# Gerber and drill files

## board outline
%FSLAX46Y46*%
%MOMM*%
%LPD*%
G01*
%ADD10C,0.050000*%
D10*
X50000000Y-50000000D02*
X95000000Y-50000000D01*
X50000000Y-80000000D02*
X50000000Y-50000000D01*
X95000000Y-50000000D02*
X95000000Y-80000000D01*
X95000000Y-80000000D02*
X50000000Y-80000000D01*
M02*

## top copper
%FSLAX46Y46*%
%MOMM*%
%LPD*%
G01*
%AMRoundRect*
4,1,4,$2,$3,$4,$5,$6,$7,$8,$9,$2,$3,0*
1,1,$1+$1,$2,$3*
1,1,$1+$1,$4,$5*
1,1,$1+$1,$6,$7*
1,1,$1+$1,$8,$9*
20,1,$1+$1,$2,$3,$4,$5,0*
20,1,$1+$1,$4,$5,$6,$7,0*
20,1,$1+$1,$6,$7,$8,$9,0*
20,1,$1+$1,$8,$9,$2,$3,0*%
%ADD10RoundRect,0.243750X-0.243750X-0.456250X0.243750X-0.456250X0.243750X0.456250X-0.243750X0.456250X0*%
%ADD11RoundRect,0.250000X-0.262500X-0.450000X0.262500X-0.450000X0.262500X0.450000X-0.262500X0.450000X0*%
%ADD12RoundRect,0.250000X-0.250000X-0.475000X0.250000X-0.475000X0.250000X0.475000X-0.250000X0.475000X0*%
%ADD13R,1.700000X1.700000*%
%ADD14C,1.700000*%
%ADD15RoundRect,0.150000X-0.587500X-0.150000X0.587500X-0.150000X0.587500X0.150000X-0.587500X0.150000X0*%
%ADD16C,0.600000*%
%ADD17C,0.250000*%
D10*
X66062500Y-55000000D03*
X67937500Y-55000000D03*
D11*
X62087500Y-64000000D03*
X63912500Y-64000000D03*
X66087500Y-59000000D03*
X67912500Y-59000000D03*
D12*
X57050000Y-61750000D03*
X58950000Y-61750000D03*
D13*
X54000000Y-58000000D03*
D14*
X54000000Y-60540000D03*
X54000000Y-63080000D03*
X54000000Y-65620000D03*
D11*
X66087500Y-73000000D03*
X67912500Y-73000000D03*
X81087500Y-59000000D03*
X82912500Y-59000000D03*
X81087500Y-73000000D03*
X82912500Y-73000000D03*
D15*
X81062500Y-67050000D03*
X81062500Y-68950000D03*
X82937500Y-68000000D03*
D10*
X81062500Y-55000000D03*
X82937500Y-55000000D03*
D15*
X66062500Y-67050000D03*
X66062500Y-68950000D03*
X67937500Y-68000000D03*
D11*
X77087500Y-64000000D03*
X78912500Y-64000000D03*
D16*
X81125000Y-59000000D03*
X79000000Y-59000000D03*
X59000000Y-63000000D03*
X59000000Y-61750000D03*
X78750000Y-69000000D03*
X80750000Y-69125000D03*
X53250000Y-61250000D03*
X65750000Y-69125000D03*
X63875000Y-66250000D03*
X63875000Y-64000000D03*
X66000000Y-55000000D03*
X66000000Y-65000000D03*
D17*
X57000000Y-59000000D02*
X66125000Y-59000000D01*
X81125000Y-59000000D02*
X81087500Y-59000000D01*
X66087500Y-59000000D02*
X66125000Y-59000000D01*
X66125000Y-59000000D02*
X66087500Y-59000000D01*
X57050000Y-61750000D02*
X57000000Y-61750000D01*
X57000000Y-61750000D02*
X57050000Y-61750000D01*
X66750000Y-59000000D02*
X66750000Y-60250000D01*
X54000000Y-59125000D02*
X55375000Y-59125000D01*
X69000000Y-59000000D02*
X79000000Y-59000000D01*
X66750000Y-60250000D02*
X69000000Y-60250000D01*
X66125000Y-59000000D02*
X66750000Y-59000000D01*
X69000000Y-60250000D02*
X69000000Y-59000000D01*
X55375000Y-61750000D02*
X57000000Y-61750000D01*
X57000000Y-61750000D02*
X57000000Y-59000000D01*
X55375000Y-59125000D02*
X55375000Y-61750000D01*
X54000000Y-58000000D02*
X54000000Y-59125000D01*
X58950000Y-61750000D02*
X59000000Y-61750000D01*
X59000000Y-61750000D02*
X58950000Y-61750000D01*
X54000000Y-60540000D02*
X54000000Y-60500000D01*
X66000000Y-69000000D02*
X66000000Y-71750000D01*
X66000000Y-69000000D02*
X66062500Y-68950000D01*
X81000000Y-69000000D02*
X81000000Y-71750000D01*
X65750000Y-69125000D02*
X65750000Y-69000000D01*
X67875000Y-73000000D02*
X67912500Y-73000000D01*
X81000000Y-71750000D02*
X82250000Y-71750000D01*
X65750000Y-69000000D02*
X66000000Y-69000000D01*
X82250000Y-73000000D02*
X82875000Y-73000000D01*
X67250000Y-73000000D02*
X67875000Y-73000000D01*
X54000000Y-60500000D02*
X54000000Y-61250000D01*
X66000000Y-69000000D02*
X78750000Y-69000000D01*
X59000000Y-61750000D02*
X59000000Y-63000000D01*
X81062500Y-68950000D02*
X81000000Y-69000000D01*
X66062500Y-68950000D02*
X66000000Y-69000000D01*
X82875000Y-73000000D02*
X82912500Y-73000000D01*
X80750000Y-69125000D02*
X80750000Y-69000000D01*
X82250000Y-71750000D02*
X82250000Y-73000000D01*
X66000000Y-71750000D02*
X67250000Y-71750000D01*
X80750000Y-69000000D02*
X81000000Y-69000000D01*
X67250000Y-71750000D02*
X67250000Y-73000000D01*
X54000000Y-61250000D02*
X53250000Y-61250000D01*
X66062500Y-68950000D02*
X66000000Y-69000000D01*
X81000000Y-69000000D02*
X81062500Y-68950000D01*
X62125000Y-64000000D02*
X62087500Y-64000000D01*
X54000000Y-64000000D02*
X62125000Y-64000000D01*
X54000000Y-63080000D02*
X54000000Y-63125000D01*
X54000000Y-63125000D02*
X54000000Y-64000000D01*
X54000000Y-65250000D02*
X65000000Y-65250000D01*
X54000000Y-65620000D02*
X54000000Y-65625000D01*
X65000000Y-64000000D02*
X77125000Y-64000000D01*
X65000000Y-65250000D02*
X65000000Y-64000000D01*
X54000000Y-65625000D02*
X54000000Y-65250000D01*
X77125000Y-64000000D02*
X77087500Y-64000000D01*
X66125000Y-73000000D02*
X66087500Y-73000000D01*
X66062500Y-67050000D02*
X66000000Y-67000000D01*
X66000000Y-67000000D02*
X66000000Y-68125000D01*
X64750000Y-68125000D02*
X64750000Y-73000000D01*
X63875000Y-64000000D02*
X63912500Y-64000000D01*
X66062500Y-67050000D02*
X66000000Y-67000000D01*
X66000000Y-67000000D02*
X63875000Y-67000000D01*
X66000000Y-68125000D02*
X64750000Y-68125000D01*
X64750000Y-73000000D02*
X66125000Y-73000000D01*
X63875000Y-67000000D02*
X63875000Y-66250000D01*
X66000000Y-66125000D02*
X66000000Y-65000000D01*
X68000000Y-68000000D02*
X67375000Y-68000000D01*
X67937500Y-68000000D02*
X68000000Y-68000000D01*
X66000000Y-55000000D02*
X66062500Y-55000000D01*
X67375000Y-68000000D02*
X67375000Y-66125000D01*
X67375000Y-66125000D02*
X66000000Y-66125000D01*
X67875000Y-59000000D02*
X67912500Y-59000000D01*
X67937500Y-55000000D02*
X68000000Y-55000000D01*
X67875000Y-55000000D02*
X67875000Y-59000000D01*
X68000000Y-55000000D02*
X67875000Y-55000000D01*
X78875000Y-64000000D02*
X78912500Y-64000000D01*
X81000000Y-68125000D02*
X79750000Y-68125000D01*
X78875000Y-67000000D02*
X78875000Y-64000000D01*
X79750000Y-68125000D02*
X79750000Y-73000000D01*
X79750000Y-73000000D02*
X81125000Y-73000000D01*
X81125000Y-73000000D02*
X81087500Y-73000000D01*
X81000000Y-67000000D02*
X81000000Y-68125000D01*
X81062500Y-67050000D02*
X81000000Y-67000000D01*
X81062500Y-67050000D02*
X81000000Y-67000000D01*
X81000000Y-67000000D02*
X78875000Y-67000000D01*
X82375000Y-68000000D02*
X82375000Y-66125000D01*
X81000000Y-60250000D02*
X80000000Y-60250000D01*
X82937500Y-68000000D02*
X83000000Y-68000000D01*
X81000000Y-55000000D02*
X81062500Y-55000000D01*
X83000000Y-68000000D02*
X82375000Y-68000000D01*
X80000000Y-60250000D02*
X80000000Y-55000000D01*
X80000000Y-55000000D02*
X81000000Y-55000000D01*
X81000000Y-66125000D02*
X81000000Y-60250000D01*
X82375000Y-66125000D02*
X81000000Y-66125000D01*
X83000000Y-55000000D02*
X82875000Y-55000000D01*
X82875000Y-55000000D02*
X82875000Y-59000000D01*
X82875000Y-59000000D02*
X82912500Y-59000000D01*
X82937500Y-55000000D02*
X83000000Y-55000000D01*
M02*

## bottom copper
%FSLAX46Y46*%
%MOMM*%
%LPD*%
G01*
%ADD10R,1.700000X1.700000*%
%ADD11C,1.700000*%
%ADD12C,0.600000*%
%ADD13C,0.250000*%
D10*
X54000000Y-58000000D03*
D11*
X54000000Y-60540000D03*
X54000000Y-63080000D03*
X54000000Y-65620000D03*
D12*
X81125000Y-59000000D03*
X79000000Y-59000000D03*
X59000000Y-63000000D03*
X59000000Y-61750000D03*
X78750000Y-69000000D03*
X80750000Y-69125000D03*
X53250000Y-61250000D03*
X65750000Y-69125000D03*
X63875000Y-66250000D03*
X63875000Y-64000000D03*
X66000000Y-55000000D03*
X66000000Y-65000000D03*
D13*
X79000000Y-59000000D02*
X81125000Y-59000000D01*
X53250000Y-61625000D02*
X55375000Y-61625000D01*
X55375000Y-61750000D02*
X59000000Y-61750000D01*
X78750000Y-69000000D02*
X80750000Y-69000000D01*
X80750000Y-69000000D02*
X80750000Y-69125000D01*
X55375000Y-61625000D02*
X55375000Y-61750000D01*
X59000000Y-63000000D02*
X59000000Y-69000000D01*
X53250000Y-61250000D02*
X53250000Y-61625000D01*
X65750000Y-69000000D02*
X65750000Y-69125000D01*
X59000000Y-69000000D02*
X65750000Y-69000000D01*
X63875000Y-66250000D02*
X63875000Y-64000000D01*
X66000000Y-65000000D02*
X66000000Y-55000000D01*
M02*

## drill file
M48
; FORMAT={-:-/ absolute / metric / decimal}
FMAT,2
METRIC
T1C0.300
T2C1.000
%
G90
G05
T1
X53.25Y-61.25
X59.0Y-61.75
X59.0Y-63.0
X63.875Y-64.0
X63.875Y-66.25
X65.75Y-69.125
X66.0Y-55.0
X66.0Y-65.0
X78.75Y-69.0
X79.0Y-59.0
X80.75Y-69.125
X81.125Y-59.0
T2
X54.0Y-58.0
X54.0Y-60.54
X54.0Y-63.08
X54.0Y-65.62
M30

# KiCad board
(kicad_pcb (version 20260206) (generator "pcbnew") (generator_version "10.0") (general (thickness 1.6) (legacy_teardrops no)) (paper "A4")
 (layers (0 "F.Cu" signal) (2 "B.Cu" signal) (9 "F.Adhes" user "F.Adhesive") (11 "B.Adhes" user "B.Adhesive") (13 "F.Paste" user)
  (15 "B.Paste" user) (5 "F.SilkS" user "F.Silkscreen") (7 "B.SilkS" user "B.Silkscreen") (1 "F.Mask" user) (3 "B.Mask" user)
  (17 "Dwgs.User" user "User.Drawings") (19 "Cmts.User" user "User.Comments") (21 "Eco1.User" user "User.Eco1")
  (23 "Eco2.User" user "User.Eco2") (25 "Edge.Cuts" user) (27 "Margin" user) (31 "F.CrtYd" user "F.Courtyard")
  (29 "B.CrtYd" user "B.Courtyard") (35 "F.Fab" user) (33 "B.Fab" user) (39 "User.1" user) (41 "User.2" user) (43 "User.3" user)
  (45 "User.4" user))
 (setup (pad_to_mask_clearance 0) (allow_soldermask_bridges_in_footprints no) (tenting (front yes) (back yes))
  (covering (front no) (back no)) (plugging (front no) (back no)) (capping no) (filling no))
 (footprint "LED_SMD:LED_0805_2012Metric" (layer "F.Cu") (at 67 55)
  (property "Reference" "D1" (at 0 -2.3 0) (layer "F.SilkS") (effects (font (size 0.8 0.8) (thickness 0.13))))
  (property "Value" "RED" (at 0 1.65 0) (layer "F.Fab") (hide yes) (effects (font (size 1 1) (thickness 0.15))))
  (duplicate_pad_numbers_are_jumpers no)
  (pad "1" smd roundrect (at -0.9375 0) (size 0.975 1.4) (layers "F.Cu" "F.Mask" "F.Paste") (roundrect_rratio 0.25) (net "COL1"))
  (pad "2" smd roundrect (at 0.9375 0) (size 0.975 1.4) (layers "F.Cu" "F.Mask" "F.Paste") (roundrect_rratio 0.25) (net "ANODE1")))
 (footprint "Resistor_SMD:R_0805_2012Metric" (layer "F.Cu") (at 63 64)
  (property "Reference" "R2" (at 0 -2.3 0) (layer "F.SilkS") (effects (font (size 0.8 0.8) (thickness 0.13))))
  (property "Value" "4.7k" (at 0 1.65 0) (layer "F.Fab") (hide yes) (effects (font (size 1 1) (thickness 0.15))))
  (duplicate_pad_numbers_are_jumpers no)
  (pad "1" smd roundrect (at -0.9125 0) (size 1.025 1.4) (layers "F.Cu" "F.Mask" "F.Paste") (roundrect_rratio 0.243902) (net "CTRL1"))
  (pad "2" smd roundrect (at 0.9125 0) (size 1.025 1.4) (layers "F.Cu" "F.Mask" "F.Paste") (roundrect_rratio 0.243902) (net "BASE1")))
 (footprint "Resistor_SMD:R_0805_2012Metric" (layer "F.Cu") (at 67 59)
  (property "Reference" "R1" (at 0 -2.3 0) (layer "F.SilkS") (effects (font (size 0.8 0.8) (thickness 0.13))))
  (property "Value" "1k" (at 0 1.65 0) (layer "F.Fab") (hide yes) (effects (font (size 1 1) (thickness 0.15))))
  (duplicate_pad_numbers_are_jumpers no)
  (pad "1" smd roundrect (at -0.9125 0) (size 1.025 1.4) (layers "F.Cu" "F.Mask" "F.Paste") (roundrect_rratio 0.243902) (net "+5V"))
  (pad "2" smd roundrect (at 0.9125 0) (size 1.025 1.4) (layers "F.Cu" "F.Mask" "F.Paste") (roundrect_rratio 0.243902) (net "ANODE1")))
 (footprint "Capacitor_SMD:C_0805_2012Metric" (layer "F.Cu") (at 58 61.75)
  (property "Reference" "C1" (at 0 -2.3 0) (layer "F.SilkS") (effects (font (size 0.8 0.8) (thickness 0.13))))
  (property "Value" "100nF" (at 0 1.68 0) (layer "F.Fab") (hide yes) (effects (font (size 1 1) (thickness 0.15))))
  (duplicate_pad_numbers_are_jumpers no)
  (pad "1" smd roundrect (at -0.95 0) (size 1 1.45) (layers "F.Cu" "F.Mask" "F.Paste") (roundrect_rratio 0.25) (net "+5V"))
  (pad "2" smd roundrect (at 0.95 0) (size 1 1.45) (layers "F.Cu" "F.Mask" "F.Paste") (roundrect_rratio 0.25) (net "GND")))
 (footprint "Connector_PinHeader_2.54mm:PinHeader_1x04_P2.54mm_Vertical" (layer "F.Cu") (at 54 58)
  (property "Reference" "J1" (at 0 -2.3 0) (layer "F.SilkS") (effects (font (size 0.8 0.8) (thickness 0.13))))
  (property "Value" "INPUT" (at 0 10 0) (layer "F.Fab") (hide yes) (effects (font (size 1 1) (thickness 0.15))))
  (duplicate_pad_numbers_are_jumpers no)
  (pad "1" thru_hole rect (at 0 0) (size 1.7 1.7) (drill 1) (layers "*.Cu" "*.Mask") (remove_unused_layers no) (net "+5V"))
  (pad "2" thru_hole circle (at 0 2.54) (size 1.7 1.7) (drill 1) (layers "*.Cu" "*.Mask") (remove_unused_layers no) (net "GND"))
  (pad "3" thru_hole circle (at 0 5.08) (size 1.7 1.7) (drill 1) (layers "*.Cu" "*.Mask") (remove_unused_layers no) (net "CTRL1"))
  (pad "4" thru_hole circle (at 0 7.62) (size 1.7 1.7) (drill 1) (layers "*.Cu" "*.Mask") (remove_unused_layers no) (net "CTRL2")))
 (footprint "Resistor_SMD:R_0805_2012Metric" (layer "F.Cu") (at 67 73)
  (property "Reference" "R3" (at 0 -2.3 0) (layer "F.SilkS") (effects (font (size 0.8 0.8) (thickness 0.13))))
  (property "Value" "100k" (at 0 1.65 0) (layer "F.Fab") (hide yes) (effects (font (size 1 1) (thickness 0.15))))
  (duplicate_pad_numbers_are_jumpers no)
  (pad "1" smd roundrect (at -0.9125 0) (size 1.025 1.4) (layers "F.Cu" "F.Mask" "F.Paste") (roundrect_rratio 0.243902) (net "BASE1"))
  (pad "2" smd roundrect (at 0.9125 0) (size 1.025 1.4) (layers "F.Cu" "F.Mask" "F.Paste") (roundrect_rratio 0.243902) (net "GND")))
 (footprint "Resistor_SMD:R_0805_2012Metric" (layer "F.Cu") (at 82 59)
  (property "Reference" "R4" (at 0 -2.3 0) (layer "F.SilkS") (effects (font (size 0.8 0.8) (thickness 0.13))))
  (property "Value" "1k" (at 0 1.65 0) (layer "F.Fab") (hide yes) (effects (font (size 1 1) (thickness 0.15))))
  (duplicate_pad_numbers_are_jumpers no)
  (pad "1" smd roundrect (at -0.9125 0) (size 1.025 1.4) (layers "F.Cu" "F.Mask" "F.Paste") (roundrect_rratio 0.243902) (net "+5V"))
  (pad "2" smd roundrect (at 0.9125 0) (size 1.025 1.4) (layers "F.Cu" "F.Mask" "F.Paste") (roundrect_rratio 0.243902) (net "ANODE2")))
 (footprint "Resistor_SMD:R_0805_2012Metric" (layer "F.Cu") (at 82 73)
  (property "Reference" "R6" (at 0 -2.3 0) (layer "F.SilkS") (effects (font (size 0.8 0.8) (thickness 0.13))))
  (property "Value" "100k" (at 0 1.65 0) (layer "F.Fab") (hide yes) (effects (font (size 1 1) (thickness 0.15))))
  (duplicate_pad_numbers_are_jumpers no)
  (pad "1" smd roundrect (at -0.9125 0) (size 1.025 1.4) (layers "F.Cu" "F.Mask" "F.Paste") (roundrect_rratio 0.243902) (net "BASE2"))
  (pad "2" smd roundrect (at 0.9125 0) (size 1.025 1.4) (layers "F.Cu" "F.Mask" "F.Paste") (roundrect_rratio 0.243902) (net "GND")))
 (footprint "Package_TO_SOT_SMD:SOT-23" (layer "F.Cu") (at 82 68)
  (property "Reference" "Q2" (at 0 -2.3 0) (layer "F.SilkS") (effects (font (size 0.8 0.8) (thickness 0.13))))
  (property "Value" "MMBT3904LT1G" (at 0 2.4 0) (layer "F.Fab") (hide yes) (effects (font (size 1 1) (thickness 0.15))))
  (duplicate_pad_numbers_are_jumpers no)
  (pad "1" smd roundrect (at -0.9375 -0.95) (size 1.475 0.6) (layers "F.Cu" "F.Mask" "F.Paste") (roundrect_rratio 0.25) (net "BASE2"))
  (pad "2" smd roundrect (at -0.9375 0.95) (size 1.475 0.6) (layers "F.Cu" "F.Mask" "F.Paste") (roundrect_rratio 0.25) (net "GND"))
  (pad "3" smd roundrect (at 0.9375 0) (size 1.475 0.6) (layers "F.Cu" "F.Mask" "F.Paste") (roundrect_rratio 0.25) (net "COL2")))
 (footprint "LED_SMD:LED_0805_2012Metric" (layer "F.Cu") (at 82 55)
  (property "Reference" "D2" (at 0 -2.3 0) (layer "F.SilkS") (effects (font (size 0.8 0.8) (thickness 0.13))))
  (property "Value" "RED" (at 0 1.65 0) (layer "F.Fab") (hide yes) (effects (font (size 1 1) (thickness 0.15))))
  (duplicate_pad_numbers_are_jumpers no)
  (pad "1" smd roundrect (at -0.9375 0) (size 0.975 1.4) (layers "F.Cu" "F.Mask" "F.Paste") (roundrect_rratio 0.25) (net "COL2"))
  (pad "2" smd roundrect (at 0.9375 0) (size 0.975 1.4) (layers "F.Cu" "F.Mask" "F.Paste") (roundrect_rratio 0.25) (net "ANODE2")))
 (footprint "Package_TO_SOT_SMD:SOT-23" (layer "F.Cu") (at 67 68)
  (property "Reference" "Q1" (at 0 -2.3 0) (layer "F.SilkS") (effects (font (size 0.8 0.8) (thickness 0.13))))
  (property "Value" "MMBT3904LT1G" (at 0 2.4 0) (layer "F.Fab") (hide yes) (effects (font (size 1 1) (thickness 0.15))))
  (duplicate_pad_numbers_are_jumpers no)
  (pad "1" smd roundrect (at -0.9375 -0.95) (size 1.475 0.6) (layers "F.Cu" "F.Mask" "F.Paste") (roundrect_rratio 0.25) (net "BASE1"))
  (pad "2" smd roundrect (at -0.9375 0.95) (size 1.475 0.6) (layers "F.Cu" "F.Mask" "F.Paste") (roundrect_rratio 0.25) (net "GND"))
  (pad "3" smd roundrect (at 0.9375 0) (size 1.475 0.6) (layers "F.Cu" "F.Mask" "F.Paste") (roundrect_rratio 0.25) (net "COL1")))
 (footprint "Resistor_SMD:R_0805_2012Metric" (layer "F.Cu") (at 78 64)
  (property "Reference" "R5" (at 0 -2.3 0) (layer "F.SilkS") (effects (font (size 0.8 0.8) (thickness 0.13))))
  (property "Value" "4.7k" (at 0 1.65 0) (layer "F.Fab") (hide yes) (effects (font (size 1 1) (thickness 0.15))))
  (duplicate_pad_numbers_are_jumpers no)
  (pad "1" smd roundrect (at -0.9125 0) (size 1.025 1.4) (layers "F.Cu" "F.Mask" "F.Paste") (roundrect_rratio 0.243902) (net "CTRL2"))
  (pad "2" smd roundrect (at 0.9125 0) (size 1.025 1.4) (layers "F.Cu" "F.Mask" "F.Paste") (roundrect_rratio 0.243902) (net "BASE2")))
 (gr_line (start 50 50) (end 95 50) (stroke (width 0.05) (type default)) (layer "Edge.Cuts"))
 (gr_line (start 50 80) (end 50 50) (stroke (width 0.05) (type default)) (layer "Edge.Cuts"))
 (gr_line (start 95 50) (end 95 80) (stroke (width 0.05) (type default)) (layer "Edge.Cuts"))
 (gr_line (start 95 80) (end 50 80) (stroke (width 0.05) (type default)) (layer "Edge.Cuts"))
 (segment (start 57 59) (end 66.125 59) (width 0.25) (layer "F.Cu") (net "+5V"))
 (segment (start 81.125 59) (end 81.0875 59) (width 0.25) (layer "F.Cu") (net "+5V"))
 (segment (start 66.0875 59) (end 66.125 59) (width 0.25) (layer "F.Cu") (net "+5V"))
 (segment (start 66.125 59) (end 66.0875 59) (width 0.25) (layer "F.Cu") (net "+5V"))
 (segment (start 57.05 61.75) (end 57 61.75) (width 0.25) (layer "F.Cu") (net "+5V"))
 (segment (start 57 61.75) (end 57.05 61.75) (width 0.25) (layer "F.Cu") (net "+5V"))
 (segment (start 66.75 59) (end 66.75 60.25) (width 0.25) (layer "F.Cu") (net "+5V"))
 (segment (start 54 59.125) (end 55.375 59.125) (width 0.25) (layer "F.Cu") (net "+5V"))
 (segment (start 69 59) (end 79 59) (width 0.25) (layer "F.Cu") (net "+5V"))
 (segment (start 66.75 60.25) (end 69 60.25) (width 0.25) (layer "F.Cu") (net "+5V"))
 (segment (start 66.125 59) (end 66.75 59) (width 0.25) (layer "F.Cu") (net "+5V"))
 (segment (start 69 60.25) (end 69 59) (width 0.25) (layer "F.Cu") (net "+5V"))
 (segment (start 55.375 61.75) (end 57 61.75) (width 0.25) (layer "F.Cu") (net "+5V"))
 (segment (start 57 61.75) (end 57 59) (width 0.25) (layer "F.Cu") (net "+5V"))
 (segment (start 55.375 59.125) (end 55.375 61.75) (width 0.25) (layer "F.Cu") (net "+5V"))
 (segment (start 54 58) (end 54 59.125) (width 0.25) (layer "F.Cu") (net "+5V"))
 (via (at 81.125 59) (size 0.6) (drill 0.3) (layers "F.Cu" "B.Cu") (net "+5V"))
 (via (at 79 59) (size 0.6) (drill 0.3) (layers "F.Cu" "B.Cu") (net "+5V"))
 (segment (start 79 59) (end 81.125 59) (width 0.25) (layer "B.Cu") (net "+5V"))
 (segment (start 58.95 61.75) (end 59 61.75) (width 0.25) (layer "F.Cu") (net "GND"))
 (segment (start 59 61.75) (end 58.95 61.75) (width 0.25) (layer "F.Cu") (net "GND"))
 (segment (start 54 60.54) (end 54 60.5) (width 0.25) (layer "F.Cu") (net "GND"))
 (segment (start 66 69) (end 66 71.75) (width 0.25) (layer "F.Cu") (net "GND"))
 (segment (start 66 69) (end 66.0625 68.95) (width 0.25) (layer "F.Cu") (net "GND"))
 (segment (start 81 69) (end 81 71.75) (width 0.25) (layer "F.Cu") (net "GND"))
 (segment (start 65.75 69.125) (end 65.75 69) (width 0.25) (layer "F.Cu") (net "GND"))
 (segment (start 67.875 73) (end 67.9125 73) (width 0.25) (layer "F.Cu") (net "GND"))
 (segment (start 81 71.75) (end 82.25 71.75) (width 0.25) (layer "F.Cu") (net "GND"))
 (segment (start 65.75 69) (end 66 69) (width 0.25) (layer "F.Cu") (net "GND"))
 (segment (start 82.25 73) (end 82.875 73) (width 0.25) (layer "F.Cu") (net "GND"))
 (segment (start 67.25 73) (end 67.875 73) (width 0.25) (layer "F.Cu") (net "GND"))
 (segment (start 54 60.5) (end 54 61.25) (width 0.25) (layer "F.Cu") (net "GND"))
 (segment (start 66 69) (end 78.75 69) (width 0.25) (layer "F.Cu") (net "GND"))
 (segment (start 59 61.75) (end 59 63) (width 0.25) (layer "F.Cu") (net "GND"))
 (segment (start 81.0625 68.95) (end 81 69) (width 0.25) (layer "F.Cu") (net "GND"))
 (segment (start 66.0625 68.95) (end 66 69) (width 0.25) (layer "F.Cu") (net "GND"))
 (segment (start 82.875 73) (end 82.9125 73) (width 0.25) (layer "F.Cu") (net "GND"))
 (segment (start 80.75 69.125) (end 80.75 69) (width 0.25) (layer "F.Cu") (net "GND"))
 (segment (start 82.25 71.75) (end 82.25 73) (width 0.25) (layer "F.Cu") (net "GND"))
 (segment (start 66 71.75) (end 67.25 71.75) (width 0.25) (layer "F.Cu") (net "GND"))
 (segment (start 80.75 69) (end 81 69) (width 0.25) (layer "F.Cu") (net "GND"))
 (segment (start 67.25 71.75) (end 67.25 73) (width 0.25) (layer "F.Cu") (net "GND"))
 (segment (start 54 61.25) (end 53.25 61.25) (width 0.25) (layer "F.Cu") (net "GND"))
 (segment (start 66.0625 68.95) (end 66 69) (width 0.25) (layer "F.Cu") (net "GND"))
 (segment (start 81 69) (end 81.0625 68.95) (width 0.25) (layer "F.Cu") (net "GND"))
 (via (at 59 63) (size 0.6) (drill 0.3) (layers "F.Cu" "B.Cu") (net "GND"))
 (via (at 59 61.75) (size 0.6) (drill 0.3) (layers "F.Cu" "B.Cu") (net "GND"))
 (via (at 78.75 69) (size 0.6) (drill 0.3) (layers "F.Cu" "B.Cu") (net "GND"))
 (via (at 80.75 69.125) (size 0.6) (drill 0.3) (layers "F.Cu" "B.Cu") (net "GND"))
 (via (at 53.25 61.25) (size 0.6) (drill 0.3) (layers "F.Cu" "B.Cu") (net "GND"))
 (via (at 65.75 69.125) (size 0.6) (drill 0.3) (layers "F.Cu" "B.Cu") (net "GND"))
 (segment (start 53.25 61.625) (end 55.375 61.625) (width 0.25) (layer "B.Cu") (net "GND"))
 (segment (start 55.375 61.75) (end 59 61.75) (width 0.25) (layer "B.Cu") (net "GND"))
 (segment (start 78.75 69) (end 80.75 69) (width 0.25) (layer "B.Cu") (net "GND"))
 (segment (start 80.75 69) (end 80.75 69.125) (width 0.25) (layer "B.Cu") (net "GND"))
 (segment (start 55.375 61.625) (end 55.375 61.75) (width 0.25) (layer "B.Cu") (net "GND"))
 (segment (start 59 63) (end 59 69) (width 0.25) (layer "B.Cu") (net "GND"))
 (segment (start 53.25 61.25) (end 53.25 61.625) (width 0.25) (layer "B.Cu") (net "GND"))
 (segment (start 65.75 69) (end 65.75 69.125) (width 0.25) (layer "B.Cu") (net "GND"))
 (segment (start 59 69) (end 65.75 69) (width 0.25) (layer "B.Cu") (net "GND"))
 (segment (start 62.125 64) (end 62.0875 64) (width 0.25) (layer "F.Cu") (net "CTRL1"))
 (segment (start 54 64) (end 62.125 64) (width 0.25) (layer "F.Cu") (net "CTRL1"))
 (segment (start 54 63.08) (end 54 63.125) (width 0.25) (layer "F.Cu") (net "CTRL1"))
 (segment (start 54 63.125) (end 54 64) (width 0.25) (layer "F.Cu") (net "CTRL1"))
 (segment (start 54 65.25) (end 65 65.25) (width 0.25) (layer "F.Cu") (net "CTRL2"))
 (segment (start 54 65.62) (end 54 65.625) (width 0.25) (layer "F.Cu") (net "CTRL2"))
 (segment (start 65 64) (end 77.125 64) (width 0.25) (layer "F.Cu") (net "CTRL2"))
 (segment (start 65 65.25) (end 65 64) (width 0.25) (layer "F.Cu") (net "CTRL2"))
 (segment (start 54 65.625) (end 54 65.25) (width 0.25) (layer "F.Cu") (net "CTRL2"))
 (segment (start 77.125 64) (end 77.0875 64) (width 0.25) (layer "F.Cu") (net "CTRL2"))
 (segment (start 66.125 73) (end 66.0875 73) (width 0.25) (layer "F.Cu") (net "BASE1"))
 (segment (start 66.0625 67.05) (end 66 67) (width 0.25) (layer "F.Cu") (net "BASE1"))
 (segment (start 66 67) (end 66 68.125) (width 0.25) (layer "F.Cu") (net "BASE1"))
 (segment (start 64.75 68.125) (end 64.75 73) (width 0.25) (layer "F.Cu") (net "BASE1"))
 (segment (start 63.875 64) (end 63.9125 64) (width 0.25) (layer "F.Cu") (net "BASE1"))
 (segment (start 66.0625 67.05) (end 66 67) (width 0.25) (layer "F.Cu") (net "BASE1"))
 (segment (start 66 67) (end 63.875 67) (width 0.25) (layer "F.Cu") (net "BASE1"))
 (segment (start 66 68.125) (end 64.75 68.125) (width 0.25) (layer "F.Cu") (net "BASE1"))
 (segment (start 64.75 73) (end 66.125 73) (width 0.25) (layer "F.Cu") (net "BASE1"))
 (segment (start 63.875 67) (end 63.875 66.25) (width 0.25) (layer "F.Cu") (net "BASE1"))
 (via (at 63.875 66.25) (size 0.6) (drill 0.3) (layers "F.Cu" "B.Cu") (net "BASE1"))
 (via (at 63.875 64) (size 0.6) (drill 0.3) (layers "F.Cu" "B.Cu") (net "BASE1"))
 (segment (start 63.875 66.25) (end 63.875 64) (width 0.25) (layer "B.Cu") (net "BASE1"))
 (segment (start 66 66.125) (end 66 65) (width 0.25) (layer "F.Cu") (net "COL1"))
 (segment (start 68 68) (end 67.375 68) (width 0.25) (layer "F.Cu") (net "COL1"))
 (segment (start 67.9375 68) (end 68 68) (width 0.25) (layer "F.Cu") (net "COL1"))
 (segment (start 66 55) (end 66.0625 55) (width 0.25) (layer "F.Cu") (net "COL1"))
 (segment (start 67.375 68) (end 67.375 66.125) (width 0.25) (layer "F.Cu") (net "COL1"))
 (segment (start 67.375 66.125) (end 66 66.125) (width 0.25) (layer "F.Cu") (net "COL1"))
 (via (at 66 55) (size 0.6) (drill 0.3) (layers "F.Cu" "B.Cu") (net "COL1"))
 (via (at 66 65) (size 0.6) (drill 0.3) (layers "F.Cu" "B.Cu") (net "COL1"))
 (segment (start 66 65) (end 66 55) (width 0.25) (layer "B.Cu") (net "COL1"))
 (segment (start 67.875 59) (end 67.9125 59) (width 0.25) (layer "F.Cu") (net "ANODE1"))
 (segment (start 67.9375 55) (end 68 55) (width 0.25) (layer "F.Cu") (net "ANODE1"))
 (segment (start 67.875 55) (end 67.875 59) (width 0.25) (layer "F.Cu") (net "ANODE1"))
 (segment (start 68 55) (end 67.875 55) (width 0.25) (layer "F.Cu") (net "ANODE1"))
 (segment (start 78.875 64) (end 78.9125 64) (width 0.25) (layer "F.Cu") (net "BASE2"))
 (segment (start 81 68.125) (end 79.75 68.125) (width 0.25) (layer "F.Cu") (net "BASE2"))
 (segment (start 78.875 67) (end 78.875 64) (width 0.25) (layer "F.Cu") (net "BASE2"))
 (segment (start 79.75 68.125) (end 79.75 73) (width 0.25) (layer "F.Cu") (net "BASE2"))
 (segment (start 79.75 73) (end 81.125 73) (width 0.25) (layer "F.Cu") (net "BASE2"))
 (segment (start 81.125 73) (end 81.0875 73) (width 0.25) (layer "F.Cu") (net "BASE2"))
 (segment (start 81 67) (end 81 68.125) (width 0.25) (layer "F.Cu") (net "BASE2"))
 (segment (start 81.0625 67.05) (end 81 67) (width 0.25) (layer "F.Cu") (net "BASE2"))
 (segment (start 81.0625 67.05) (end 81 67) (width 0.25) (layer "F.Cu") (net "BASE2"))
 (segment (start 81 67) (end 78.875 67) (width 0.25) (layer "F.Cu") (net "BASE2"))
 (segment (start 82.375 68) (end 82.375 66.125) (width 0.25) (layer "F.Cu") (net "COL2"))
 (segment (start 81 60.25) (end 80 60.25) (width 0.25) (layer "F.Cu") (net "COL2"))
 (segment (start 82.9375 68) (end 83 68) (width 0.25) (layer "F.Cu") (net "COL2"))
 (segment (start 81 55) (end 81.0625 55) (width 0.25) (layer "F.Cu") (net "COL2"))
 (segment (start 83 68) (end 82.375 68) (width 0.25) (layer "F.Cu") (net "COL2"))
 (segment (start 80 60.25) (end 80 55) (width 0.25) (layer "F.Cu") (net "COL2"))
 (segment (start 80 55) (end 81 55) (width 0.25) (layer "F.Cu") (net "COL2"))
 (segment (start 81 66.125) (end 81 60.25) (width 0.25) (layer "F.Cu") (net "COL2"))
 (segment (start 82.375 66.125) (end 81 66.125) (width 0.25) (layer "F.Cu") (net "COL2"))
 (segment (start 83 55) (end 82.875 55) (width 0.25) (layer "F.Cu") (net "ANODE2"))
 (segment (start 82.875 55) (end 82.875 59) (width 0.25) (layer "F.Cu") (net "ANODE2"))
 (segment (start 82.875 59) (end 82.9125 59) (width 0.25) (layer "F.Cu") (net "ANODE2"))
 (segment (start 82.9375 55) (end 83 55) (width 0.25) (layer "F.Cu") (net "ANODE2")))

